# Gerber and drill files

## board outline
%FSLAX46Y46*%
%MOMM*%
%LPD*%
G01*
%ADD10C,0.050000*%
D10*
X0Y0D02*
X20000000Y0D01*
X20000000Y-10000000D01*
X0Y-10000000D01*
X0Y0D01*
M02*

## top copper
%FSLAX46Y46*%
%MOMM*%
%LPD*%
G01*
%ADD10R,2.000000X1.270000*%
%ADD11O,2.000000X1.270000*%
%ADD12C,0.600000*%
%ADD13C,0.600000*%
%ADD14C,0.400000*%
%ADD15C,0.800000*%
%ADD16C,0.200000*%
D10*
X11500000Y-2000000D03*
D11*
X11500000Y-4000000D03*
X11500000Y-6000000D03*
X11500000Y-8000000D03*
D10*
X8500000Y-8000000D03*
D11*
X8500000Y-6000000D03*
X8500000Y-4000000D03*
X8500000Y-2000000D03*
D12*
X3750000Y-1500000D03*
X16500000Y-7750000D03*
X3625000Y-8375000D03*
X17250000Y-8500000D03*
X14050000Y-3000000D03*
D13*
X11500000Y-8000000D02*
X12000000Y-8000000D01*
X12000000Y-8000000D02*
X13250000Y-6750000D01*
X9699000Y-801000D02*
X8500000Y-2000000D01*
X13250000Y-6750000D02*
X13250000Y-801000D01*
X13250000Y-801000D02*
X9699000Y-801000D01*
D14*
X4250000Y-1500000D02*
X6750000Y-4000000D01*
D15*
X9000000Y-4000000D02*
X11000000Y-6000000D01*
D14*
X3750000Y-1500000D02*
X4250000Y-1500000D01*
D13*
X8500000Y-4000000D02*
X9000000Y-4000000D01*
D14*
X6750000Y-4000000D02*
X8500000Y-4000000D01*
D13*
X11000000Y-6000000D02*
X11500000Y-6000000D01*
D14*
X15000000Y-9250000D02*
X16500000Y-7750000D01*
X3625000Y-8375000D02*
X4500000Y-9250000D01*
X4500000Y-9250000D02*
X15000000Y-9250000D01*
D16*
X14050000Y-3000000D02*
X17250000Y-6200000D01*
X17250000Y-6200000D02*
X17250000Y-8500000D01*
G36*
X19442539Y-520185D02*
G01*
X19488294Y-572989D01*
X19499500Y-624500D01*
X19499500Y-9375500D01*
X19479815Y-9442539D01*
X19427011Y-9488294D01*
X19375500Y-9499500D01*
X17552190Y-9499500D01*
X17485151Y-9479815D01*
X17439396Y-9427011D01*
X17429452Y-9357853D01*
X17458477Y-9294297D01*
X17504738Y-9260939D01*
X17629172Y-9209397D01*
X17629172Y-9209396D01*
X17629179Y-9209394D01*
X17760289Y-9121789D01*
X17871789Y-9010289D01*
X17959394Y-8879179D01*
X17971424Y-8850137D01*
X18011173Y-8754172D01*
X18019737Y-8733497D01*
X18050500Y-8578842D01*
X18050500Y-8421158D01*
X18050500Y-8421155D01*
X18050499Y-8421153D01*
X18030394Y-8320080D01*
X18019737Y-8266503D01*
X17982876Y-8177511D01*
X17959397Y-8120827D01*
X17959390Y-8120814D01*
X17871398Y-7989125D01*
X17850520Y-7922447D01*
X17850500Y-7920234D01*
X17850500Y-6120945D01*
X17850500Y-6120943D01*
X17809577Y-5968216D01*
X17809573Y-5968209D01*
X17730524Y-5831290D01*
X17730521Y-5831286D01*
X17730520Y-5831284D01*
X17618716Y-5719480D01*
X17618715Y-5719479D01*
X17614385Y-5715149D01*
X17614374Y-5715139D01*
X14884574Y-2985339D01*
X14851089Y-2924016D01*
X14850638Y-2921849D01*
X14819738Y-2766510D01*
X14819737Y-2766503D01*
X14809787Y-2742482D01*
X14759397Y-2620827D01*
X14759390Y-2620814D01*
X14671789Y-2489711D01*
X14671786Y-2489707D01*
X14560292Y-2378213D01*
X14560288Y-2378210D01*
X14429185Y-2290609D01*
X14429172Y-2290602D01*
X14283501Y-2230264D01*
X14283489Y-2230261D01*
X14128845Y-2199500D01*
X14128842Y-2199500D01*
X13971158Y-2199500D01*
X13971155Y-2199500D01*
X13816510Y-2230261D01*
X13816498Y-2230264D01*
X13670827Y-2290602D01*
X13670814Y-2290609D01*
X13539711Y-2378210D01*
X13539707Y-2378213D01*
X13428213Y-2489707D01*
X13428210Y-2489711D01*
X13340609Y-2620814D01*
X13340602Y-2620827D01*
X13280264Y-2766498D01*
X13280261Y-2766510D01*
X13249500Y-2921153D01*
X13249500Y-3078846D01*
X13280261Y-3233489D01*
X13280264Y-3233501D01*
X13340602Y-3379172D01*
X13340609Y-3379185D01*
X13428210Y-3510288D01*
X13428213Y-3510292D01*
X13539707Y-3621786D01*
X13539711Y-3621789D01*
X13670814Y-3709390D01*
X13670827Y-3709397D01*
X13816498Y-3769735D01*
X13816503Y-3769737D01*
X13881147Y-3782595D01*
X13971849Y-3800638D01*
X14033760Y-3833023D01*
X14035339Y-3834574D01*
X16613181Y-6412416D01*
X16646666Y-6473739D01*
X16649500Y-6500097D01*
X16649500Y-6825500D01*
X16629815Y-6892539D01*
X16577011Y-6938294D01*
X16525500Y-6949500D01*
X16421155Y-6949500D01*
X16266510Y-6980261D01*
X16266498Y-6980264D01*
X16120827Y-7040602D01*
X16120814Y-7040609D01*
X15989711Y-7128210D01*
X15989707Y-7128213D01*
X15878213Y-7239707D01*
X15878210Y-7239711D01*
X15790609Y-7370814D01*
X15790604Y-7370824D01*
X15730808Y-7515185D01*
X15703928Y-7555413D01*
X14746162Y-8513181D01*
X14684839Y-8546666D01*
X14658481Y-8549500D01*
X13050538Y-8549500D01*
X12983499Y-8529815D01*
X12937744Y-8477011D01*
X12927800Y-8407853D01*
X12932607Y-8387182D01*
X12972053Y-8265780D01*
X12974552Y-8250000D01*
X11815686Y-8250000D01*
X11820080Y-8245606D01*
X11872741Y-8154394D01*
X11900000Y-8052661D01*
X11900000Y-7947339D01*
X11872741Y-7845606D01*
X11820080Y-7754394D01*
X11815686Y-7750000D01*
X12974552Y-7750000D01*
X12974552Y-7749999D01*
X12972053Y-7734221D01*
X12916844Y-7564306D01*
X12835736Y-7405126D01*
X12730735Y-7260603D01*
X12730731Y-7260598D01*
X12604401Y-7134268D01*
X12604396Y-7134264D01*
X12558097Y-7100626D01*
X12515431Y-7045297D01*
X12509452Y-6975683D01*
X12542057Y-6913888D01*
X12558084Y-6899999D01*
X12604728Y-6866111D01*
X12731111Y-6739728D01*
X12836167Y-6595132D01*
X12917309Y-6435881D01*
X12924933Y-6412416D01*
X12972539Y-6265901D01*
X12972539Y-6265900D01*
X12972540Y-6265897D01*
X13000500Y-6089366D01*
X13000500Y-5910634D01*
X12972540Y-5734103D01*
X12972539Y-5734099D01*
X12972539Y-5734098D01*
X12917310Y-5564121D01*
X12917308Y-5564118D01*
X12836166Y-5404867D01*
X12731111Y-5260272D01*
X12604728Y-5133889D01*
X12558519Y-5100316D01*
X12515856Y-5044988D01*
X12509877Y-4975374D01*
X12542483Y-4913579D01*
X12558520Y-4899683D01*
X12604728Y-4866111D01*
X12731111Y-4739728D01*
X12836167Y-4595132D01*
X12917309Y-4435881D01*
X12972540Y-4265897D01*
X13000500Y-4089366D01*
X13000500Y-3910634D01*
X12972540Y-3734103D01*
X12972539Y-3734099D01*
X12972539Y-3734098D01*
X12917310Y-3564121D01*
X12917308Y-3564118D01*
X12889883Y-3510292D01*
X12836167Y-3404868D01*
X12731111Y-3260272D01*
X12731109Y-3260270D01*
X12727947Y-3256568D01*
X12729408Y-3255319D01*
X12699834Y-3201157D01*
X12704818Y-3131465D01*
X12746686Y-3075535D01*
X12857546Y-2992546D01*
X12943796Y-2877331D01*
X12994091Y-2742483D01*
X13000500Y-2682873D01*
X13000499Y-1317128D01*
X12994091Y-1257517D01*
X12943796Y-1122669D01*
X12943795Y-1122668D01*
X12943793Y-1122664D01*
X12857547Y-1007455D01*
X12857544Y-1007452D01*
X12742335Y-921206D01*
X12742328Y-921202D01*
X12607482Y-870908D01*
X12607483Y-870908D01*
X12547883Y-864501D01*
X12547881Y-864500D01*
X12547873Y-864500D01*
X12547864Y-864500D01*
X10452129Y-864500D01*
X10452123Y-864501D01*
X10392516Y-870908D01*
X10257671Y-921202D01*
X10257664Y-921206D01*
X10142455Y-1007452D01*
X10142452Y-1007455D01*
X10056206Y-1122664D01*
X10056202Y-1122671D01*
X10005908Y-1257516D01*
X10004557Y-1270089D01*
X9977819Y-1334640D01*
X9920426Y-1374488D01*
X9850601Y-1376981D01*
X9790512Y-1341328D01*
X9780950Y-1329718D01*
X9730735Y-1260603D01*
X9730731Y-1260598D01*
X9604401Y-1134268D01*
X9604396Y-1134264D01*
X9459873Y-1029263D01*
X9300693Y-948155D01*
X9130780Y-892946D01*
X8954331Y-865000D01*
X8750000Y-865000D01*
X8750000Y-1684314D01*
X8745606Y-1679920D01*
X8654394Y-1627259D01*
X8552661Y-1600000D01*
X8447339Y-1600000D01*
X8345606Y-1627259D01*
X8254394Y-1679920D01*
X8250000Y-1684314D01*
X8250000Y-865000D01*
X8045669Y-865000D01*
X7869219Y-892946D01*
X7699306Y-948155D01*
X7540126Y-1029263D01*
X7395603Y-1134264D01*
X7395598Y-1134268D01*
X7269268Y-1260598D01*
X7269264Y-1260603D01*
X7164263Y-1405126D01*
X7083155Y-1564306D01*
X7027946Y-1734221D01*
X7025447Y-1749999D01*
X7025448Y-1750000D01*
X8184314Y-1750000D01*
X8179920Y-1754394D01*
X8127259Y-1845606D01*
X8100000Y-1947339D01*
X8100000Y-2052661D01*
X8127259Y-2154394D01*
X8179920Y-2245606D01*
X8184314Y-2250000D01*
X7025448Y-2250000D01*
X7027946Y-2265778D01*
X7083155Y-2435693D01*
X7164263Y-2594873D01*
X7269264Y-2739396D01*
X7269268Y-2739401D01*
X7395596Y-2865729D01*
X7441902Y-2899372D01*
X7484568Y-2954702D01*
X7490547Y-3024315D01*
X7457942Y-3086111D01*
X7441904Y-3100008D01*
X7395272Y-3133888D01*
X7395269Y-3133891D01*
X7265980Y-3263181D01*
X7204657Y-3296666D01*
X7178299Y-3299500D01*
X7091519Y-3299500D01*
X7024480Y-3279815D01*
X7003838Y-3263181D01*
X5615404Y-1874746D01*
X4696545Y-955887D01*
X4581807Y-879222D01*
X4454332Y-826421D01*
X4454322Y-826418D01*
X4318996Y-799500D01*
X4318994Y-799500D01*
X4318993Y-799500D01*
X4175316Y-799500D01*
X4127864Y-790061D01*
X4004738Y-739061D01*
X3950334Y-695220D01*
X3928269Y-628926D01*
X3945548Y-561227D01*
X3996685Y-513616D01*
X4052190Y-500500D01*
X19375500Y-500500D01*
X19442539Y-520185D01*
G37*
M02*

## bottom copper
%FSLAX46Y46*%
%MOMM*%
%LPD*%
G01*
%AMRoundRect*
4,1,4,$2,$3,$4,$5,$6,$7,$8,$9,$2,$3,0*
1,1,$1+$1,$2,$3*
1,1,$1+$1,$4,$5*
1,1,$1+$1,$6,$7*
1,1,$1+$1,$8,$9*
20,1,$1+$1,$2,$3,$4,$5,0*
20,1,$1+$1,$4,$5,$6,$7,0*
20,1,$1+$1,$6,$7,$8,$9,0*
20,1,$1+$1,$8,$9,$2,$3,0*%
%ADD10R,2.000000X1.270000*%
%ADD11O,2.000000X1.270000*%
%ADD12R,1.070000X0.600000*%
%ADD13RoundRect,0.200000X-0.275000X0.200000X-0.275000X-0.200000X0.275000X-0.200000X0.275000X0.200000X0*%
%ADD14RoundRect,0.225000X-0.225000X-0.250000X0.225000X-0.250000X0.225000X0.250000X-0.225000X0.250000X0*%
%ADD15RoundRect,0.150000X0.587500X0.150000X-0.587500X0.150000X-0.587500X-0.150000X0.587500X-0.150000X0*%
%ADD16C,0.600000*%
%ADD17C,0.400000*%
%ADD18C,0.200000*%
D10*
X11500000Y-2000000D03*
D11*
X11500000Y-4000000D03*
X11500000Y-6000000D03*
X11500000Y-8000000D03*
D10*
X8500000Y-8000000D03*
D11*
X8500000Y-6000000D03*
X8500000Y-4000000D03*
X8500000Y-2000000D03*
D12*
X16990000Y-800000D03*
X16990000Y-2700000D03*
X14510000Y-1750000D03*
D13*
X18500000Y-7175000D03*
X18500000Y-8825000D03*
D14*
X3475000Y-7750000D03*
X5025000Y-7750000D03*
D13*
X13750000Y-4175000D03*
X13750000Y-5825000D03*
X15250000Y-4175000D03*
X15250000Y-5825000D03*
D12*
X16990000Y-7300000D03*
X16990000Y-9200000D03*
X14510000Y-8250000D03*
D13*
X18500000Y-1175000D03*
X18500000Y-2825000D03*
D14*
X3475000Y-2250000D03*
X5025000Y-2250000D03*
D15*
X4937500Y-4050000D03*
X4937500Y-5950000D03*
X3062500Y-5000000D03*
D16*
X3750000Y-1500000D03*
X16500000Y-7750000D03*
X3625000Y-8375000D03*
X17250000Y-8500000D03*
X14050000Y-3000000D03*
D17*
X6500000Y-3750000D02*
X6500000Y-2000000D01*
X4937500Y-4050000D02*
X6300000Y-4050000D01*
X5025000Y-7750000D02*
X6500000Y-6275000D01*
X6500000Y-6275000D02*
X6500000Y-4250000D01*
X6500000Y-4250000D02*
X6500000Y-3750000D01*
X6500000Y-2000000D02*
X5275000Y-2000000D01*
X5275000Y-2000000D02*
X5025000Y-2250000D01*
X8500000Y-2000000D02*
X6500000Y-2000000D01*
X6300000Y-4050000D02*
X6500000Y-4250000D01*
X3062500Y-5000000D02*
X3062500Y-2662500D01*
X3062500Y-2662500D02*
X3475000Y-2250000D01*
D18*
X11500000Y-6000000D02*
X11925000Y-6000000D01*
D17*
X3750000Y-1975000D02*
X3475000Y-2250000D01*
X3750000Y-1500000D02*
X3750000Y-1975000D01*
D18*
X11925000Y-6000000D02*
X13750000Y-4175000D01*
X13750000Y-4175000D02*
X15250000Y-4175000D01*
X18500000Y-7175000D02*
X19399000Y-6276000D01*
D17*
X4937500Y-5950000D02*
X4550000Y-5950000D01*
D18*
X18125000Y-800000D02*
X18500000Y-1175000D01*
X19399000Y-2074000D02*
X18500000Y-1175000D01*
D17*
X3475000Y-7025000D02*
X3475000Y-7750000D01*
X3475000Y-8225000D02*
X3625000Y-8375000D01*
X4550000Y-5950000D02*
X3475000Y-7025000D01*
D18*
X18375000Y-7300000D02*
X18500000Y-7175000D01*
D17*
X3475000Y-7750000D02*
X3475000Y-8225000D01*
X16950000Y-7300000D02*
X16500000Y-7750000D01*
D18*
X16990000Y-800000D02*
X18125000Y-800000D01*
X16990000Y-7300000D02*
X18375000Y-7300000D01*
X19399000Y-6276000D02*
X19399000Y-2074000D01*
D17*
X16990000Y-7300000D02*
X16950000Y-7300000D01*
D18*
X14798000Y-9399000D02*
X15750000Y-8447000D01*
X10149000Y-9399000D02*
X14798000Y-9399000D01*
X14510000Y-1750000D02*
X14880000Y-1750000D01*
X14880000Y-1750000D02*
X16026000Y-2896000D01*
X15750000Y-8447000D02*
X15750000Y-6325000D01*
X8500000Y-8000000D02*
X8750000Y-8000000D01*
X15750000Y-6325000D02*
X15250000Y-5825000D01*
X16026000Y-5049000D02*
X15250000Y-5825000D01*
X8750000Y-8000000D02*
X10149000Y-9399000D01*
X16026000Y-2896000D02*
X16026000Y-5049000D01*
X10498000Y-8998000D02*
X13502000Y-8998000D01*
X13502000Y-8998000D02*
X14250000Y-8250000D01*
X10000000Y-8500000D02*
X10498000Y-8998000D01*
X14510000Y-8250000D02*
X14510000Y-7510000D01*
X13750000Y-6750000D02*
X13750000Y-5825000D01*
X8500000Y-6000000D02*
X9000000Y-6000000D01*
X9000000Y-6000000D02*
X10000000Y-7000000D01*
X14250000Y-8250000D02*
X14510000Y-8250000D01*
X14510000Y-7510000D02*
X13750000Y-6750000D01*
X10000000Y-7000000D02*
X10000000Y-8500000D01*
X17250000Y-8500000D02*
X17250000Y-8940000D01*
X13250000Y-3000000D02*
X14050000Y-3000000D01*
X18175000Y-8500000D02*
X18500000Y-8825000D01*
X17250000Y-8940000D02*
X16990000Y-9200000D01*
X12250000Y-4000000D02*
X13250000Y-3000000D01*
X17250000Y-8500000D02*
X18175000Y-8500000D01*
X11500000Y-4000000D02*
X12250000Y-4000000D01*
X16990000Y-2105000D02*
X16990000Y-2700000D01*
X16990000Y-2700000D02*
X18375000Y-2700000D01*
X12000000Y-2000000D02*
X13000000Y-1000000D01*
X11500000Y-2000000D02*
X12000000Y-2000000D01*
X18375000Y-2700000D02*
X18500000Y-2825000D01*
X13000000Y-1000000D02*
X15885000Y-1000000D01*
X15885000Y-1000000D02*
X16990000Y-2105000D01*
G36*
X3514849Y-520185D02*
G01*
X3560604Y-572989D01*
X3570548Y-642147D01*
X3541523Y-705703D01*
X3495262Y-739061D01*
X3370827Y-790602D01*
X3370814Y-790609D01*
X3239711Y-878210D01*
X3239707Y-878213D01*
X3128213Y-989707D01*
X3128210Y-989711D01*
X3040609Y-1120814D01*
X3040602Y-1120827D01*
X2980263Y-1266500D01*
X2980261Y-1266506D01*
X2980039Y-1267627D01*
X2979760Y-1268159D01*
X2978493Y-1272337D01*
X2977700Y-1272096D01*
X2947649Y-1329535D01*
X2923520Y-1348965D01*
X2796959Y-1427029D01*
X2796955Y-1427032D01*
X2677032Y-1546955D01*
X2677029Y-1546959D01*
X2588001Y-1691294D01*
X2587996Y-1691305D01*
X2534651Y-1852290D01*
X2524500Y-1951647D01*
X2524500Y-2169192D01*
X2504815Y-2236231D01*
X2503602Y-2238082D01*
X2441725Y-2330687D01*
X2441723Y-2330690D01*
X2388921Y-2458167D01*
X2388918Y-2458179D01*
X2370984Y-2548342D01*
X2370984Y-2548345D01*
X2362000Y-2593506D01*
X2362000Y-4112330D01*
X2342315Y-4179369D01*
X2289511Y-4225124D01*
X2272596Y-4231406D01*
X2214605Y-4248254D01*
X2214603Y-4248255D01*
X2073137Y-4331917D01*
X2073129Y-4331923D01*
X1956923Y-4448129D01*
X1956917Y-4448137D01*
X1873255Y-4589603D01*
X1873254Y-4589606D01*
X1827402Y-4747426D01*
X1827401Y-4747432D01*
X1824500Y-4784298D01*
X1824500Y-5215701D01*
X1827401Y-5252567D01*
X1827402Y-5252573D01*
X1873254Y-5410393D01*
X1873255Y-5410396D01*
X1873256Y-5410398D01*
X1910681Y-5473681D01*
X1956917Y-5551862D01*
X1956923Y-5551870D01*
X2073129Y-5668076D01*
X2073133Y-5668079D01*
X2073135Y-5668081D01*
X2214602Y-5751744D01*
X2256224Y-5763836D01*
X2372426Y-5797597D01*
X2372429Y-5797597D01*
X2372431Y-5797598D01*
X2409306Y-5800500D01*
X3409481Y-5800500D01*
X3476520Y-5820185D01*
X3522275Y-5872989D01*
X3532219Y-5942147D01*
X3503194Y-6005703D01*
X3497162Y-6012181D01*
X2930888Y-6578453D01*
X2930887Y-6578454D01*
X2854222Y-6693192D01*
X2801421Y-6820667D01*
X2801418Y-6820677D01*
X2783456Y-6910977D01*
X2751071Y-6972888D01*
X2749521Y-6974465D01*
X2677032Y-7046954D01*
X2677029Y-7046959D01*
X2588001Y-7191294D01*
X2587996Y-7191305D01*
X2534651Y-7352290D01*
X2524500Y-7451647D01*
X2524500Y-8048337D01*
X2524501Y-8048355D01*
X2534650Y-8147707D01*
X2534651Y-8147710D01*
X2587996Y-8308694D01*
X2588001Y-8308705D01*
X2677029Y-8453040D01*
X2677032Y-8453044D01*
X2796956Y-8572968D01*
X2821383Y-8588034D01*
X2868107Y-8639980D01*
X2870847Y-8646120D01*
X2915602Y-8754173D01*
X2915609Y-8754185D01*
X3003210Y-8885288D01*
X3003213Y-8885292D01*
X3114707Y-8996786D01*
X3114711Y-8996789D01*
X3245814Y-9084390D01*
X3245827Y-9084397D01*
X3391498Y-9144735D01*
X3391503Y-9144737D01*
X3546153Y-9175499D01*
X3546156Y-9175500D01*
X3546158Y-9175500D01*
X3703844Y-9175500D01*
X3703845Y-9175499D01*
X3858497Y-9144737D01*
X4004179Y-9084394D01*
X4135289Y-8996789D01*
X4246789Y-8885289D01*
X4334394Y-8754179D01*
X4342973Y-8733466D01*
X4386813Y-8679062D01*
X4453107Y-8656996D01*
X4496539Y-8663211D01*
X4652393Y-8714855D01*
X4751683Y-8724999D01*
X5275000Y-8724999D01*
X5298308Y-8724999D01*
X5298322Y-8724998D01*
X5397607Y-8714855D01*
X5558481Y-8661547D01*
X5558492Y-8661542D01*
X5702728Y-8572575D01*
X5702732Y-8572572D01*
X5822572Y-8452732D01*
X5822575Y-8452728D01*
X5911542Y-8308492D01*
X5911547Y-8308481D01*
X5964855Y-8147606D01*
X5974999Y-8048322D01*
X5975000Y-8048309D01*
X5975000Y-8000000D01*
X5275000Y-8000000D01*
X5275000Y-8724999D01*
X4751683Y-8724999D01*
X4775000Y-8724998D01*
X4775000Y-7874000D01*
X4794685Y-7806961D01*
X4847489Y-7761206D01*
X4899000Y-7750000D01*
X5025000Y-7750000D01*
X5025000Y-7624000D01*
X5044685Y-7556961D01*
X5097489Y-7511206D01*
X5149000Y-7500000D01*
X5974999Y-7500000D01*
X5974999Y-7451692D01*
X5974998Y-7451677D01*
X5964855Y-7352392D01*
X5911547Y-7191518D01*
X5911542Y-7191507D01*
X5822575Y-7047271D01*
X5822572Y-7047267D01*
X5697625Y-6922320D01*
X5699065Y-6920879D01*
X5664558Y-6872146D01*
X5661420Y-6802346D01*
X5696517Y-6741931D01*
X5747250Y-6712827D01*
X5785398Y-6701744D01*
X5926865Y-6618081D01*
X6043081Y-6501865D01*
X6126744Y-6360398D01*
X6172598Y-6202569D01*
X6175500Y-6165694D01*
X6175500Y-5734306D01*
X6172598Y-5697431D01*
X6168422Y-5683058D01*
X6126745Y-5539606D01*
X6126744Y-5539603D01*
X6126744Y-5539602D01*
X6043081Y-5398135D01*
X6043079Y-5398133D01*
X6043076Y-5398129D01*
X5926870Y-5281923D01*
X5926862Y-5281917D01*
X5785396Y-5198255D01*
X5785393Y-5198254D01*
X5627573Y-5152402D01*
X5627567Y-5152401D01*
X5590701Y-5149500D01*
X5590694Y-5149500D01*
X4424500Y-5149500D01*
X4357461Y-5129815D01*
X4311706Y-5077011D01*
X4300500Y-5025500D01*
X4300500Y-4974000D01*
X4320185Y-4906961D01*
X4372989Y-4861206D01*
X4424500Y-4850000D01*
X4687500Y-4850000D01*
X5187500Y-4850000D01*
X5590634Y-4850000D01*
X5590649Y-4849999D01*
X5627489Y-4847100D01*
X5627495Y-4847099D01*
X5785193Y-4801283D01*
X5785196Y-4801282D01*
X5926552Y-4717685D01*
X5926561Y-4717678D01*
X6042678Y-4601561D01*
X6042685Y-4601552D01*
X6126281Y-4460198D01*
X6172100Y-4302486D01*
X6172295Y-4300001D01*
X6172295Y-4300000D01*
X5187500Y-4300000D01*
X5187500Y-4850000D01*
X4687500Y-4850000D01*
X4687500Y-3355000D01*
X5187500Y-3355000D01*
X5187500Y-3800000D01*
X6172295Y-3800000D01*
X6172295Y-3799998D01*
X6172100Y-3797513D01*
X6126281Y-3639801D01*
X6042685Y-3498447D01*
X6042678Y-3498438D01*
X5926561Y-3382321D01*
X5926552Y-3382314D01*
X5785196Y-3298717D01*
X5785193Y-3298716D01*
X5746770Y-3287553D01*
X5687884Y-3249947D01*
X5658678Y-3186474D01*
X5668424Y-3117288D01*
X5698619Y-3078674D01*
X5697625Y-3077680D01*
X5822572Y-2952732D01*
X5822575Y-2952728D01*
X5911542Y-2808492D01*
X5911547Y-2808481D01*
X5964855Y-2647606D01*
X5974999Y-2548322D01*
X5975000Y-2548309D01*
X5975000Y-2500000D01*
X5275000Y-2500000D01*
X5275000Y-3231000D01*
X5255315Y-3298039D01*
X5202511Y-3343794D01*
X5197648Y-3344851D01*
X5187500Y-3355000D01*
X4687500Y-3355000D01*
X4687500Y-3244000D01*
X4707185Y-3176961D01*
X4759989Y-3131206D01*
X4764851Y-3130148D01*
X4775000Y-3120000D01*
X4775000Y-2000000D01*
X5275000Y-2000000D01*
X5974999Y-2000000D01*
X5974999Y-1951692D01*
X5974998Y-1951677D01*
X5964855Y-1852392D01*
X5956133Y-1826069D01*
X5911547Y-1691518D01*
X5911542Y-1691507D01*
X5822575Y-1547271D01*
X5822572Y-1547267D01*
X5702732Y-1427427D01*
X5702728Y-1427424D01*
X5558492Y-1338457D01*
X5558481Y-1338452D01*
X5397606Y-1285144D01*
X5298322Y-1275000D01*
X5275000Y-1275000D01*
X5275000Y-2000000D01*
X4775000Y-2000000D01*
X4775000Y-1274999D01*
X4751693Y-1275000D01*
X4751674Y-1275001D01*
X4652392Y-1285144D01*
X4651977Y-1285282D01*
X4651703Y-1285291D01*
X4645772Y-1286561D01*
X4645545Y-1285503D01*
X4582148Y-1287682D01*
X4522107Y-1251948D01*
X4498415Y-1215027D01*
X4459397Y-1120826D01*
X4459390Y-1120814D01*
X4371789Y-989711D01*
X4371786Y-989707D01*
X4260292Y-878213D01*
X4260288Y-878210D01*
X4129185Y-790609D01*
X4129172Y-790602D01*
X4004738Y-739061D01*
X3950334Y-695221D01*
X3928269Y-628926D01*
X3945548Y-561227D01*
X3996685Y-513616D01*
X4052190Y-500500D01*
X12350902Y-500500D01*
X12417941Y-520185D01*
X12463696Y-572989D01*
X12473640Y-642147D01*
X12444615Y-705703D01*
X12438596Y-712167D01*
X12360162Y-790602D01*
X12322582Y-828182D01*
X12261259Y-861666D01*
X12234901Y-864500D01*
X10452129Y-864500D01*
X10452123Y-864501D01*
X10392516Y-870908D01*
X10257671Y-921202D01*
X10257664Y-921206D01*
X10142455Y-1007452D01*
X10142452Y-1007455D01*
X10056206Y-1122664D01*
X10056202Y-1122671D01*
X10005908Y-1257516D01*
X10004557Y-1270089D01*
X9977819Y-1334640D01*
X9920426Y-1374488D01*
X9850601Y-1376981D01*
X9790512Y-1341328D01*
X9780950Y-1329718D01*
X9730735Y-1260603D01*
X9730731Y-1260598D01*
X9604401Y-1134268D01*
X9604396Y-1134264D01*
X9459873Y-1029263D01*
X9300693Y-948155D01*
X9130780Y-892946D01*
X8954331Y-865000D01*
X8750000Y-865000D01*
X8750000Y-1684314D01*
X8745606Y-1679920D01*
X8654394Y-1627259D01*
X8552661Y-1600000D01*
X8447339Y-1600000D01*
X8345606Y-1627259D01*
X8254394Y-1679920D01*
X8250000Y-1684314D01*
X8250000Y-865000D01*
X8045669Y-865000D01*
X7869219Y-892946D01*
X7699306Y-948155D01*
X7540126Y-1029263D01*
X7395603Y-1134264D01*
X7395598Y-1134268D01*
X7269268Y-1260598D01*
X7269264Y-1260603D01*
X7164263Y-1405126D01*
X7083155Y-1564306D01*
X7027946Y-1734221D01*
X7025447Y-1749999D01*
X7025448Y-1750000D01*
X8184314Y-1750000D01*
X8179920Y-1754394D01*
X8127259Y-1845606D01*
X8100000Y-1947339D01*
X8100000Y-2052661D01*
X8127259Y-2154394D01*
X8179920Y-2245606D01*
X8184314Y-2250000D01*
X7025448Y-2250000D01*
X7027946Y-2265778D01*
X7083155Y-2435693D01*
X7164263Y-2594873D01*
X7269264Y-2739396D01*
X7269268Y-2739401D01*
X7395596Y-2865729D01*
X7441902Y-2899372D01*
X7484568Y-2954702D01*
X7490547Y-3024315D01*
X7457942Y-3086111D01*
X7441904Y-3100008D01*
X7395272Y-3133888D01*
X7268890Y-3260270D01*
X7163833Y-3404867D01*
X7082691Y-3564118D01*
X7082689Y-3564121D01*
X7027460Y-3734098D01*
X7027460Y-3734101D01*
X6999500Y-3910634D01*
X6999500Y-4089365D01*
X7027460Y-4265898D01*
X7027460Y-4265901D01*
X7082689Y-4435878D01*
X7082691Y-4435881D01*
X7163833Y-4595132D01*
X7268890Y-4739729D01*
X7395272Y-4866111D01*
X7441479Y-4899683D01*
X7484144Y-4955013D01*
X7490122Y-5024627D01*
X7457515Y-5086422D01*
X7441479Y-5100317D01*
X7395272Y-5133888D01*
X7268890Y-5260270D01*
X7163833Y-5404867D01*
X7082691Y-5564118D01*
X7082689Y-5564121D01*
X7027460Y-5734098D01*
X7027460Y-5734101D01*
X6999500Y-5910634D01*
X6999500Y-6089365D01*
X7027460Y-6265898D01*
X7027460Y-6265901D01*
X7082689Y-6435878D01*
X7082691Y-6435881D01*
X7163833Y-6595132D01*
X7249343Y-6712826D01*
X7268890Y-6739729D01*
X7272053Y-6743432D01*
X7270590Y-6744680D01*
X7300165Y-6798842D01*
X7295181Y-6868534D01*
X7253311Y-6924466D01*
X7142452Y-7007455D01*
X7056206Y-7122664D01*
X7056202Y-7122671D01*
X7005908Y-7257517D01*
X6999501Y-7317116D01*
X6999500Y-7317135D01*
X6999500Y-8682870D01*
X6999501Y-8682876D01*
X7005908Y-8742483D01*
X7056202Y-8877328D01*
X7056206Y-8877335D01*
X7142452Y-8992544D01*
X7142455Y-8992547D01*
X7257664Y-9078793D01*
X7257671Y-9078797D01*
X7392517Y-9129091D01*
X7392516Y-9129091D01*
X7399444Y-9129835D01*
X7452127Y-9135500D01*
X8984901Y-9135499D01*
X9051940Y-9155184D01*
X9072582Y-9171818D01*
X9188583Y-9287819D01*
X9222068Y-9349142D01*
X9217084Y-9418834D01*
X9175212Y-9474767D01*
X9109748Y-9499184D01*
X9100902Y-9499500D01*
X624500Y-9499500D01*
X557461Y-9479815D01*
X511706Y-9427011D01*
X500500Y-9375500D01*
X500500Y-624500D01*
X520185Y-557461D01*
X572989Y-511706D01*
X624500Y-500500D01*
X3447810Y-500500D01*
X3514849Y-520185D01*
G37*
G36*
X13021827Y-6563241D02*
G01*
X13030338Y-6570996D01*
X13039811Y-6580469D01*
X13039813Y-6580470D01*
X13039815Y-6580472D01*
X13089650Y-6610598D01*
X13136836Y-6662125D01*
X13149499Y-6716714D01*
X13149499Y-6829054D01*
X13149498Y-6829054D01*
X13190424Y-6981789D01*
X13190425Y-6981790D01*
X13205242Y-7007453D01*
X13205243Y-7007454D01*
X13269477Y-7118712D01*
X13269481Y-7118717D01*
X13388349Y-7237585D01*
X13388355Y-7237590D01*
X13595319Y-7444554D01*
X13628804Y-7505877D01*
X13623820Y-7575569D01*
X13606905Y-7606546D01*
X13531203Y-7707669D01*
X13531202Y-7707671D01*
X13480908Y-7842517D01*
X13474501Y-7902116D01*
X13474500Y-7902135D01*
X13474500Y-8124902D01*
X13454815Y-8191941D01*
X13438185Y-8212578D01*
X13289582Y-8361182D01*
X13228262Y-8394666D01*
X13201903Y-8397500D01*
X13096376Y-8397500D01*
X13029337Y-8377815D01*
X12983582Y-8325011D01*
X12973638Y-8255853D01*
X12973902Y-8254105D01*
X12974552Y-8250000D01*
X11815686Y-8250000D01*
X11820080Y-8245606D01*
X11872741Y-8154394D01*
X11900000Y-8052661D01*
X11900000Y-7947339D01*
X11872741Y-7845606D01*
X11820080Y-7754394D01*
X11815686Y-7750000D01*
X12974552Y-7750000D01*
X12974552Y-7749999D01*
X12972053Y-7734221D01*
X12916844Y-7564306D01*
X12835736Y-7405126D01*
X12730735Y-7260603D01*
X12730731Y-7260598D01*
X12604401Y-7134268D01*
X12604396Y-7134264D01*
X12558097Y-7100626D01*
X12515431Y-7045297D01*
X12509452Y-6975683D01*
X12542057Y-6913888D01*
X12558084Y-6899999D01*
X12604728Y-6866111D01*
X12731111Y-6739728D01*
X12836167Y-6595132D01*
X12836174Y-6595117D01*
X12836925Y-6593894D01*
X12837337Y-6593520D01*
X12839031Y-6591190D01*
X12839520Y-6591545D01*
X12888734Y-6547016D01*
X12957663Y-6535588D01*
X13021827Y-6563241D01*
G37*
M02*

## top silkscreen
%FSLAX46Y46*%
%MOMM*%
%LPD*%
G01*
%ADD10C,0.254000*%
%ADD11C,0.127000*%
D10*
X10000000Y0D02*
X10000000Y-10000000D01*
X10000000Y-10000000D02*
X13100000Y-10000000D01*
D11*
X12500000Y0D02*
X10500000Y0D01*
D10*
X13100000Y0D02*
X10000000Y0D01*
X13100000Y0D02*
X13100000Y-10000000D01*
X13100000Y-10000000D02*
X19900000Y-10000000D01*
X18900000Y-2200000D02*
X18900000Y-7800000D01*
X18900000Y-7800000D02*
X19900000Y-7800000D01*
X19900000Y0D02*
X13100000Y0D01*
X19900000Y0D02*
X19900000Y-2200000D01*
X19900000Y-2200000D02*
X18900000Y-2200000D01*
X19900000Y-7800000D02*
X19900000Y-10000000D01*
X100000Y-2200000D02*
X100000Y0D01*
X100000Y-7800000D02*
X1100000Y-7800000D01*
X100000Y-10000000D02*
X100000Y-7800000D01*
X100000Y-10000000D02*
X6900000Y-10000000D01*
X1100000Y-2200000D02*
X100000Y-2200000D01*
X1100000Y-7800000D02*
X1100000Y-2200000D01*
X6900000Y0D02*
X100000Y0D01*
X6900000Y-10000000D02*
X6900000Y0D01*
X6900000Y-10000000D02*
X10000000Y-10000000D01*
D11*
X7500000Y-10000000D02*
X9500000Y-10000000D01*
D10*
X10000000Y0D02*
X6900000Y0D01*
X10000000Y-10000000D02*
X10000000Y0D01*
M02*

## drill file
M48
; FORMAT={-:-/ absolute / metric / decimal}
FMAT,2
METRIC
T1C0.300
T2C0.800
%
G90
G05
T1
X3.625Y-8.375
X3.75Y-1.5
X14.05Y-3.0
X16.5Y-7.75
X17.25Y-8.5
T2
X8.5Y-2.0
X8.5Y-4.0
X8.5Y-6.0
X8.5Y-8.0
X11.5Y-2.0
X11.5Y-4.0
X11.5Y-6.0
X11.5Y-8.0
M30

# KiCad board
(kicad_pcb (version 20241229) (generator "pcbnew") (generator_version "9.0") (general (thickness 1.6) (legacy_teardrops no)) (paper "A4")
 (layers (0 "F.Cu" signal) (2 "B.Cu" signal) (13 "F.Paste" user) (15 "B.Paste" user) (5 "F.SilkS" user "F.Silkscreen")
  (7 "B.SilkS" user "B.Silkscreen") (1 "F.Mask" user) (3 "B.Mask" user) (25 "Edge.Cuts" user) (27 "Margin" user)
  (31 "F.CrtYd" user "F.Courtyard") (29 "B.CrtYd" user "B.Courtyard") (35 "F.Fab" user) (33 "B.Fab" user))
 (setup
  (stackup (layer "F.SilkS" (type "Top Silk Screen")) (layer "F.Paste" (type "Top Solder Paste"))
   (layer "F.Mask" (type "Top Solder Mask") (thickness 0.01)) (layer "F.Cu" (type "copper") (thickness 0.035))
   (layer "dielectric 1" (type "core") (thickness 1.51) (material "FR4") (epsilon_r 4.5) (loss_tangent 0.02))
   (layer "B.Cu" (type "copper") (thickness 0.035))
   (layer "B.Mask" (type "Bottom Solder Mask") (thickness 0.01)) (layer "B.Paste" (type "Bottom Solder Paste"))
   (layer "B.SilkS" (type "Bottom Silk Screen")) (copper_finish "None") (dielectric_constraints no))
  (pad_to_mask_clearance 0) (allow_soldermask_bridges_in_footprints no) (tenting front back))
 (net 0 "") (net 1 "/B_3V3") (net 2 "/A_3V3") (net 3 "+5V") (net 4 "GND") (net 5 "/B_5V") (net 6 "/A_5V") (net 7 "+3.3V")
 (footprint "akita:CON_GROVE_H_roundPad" (layer "F.Cu") (at 11.5 5 -90)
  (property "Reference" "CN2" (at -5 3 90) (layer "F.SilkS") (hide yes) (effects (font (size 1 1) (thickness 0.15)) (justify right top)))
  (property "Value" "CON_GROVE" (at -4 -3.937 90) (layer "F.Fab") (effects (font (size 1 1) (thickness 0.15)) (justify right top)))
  (fp_line (start -5 1.5) (end 5 1.5) (stroke (width 0.254) (type solid)) (layer "F.SilkS"))
  (fp_line (start 5 1.5) (end 5 -1.6) (stroke (width 0.254) (type solid)) (layer "F.SilkS"))
  (fp_line (start -5 -1) (end -5 1) (stroke (width 0.127) (type solid)) (layer "F.SilkS"))
  (fp_line (start -5 -1.6) (end -5 1.5) (stroke (width 0.254) (type solid)) (layer "F.SilkS"))
  (fp_line (start -5 -1.6) (end 5 -1.6) (stroke (width 0.254) (type solid)) (layer "F.SilkS"))
  (fp_line (start 5 -1.6) (end 5 -8.4) (stroke (width 0.254) (type solid)) (layer "F.SilkS"))
  (fp_line (start -2.8 -7.4) (end 2.8 -7.4) (stroke (width 0.254) (type solid)) (layer "F.SilkS"))
  (fp_line (start 2.8 -7.4) (end 2.8 -8.4) (stroke (width 0.254) (type solid)) (layer "F.SilkS"))
  (fp_line (start -5 -8.4) (end -5 -1.6) (stroke (width 0.254) (type solid)) (layer "F.SilkS"))
  (fp_line (start -5 -8.4) (end -2.8 -8.4) (stroke (width 0.254) (type solid)) (layer "F.SilkS"))
  (fp_line (start -2.8 -8.4) (end -2.8 -7.4) (stroke (width 0.254) (type solid)) (layer "F.SilkS"))
  (fp_line (start 2.8 -8.4) (end 5 -8.4) (stroke (width 0.254) (type solid)) (layer "F.SilkS"))
  (pad "1" thru_hole rect (at -3 0 270) (size 1.27 2) (drill 0.8) (layers "*.Cu" "*.Mask") (remove_unused_layers no) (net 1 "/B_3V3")
   (solder_mask_margin 0.1016))
  (pad "2" thru_hole oval (at -1 0 270) (size 1.27 2) (drill 0.8) (layers "*.Cu" "*.Mask") (remove_unused_layers no) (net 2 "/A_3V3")
   (solder_mask_margin 0.1016))
  (pad "3" thru_hole oval (at 1 0 270) (size 1.27 2) (drill 0.8) (layers "*.Cu" "*.Mask") (remove_unused_layers no) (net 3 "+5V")
   (solder_mask_margin 0.1016))
  (pad "4" thru_hole oval (at 3 0 270) (size 1.27 2) (drill 0.8) (layers "*.Cu" "*.Mask") (remove_unused_layers no) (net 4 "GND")
   (solder_mask_margin 0.1016)))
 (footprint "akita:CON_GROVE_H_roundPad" (layer "F.Cu") (at 8.5 5 90)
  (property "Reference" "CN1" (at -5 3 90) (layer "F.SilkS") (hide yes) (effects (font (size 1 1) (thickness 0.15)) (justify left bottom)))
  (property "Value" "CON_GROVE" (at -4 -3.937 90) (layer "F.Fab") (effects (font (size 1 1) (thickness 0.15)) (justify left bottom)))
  (fp_line (start 2.8 -8.4) (end 5 -8.4) (stroke (width 0.254) (type solid)) (layer "F.SilkS"))
  (fp_line (start -2.8 -8.4) (end -2.8 -7.4) (stroke (width 0.254) (type solid)) (layer "F.SilkS"))
  (fp_line (start -5 -8.4) (end -2.8 -8.4) (stroke (width 0.254) (type solid)) (layer "F.SilkS"))
  (fp_line (start -5 -8.4) (end -5 -1.6) (stroke (width 0.254) (type solid)) (layer "F.SilkS"))
  (fp_line (start 2.8 -7.4) (end 2.8 -8.4) (stroke (width 0.254) (type solid)) (layer "F.SilkS"))
  (fp_line (start -2.8 -7.4) (end 2.8 -7.4) (stroke (width 0.254) (type solid)) (layer "F.SilkS"))
  (fp_line (start 5 -1.6) (end 5 -8.4) (stroke (width 0.254) (type solid)) (layer "F.SilkS"))
  (fp_line (start -5 -1.6) (end 5 -1.6) (stroke (width 0.254) (type solid)) (layer "F.SilkS"))
  (fp_line (start -5 -1.6) (end -5 1.5) (stroke (width 0.254) (type solid)) (layer "F.SilkS"))
  (fp_line (start -5 -1) (end -5 1) (stroke (width 0.127) (type solid)) (layer "F.SilkS"))
  (fp_line (start 5 1.5) (end 5 -1.6) (stroke (width 0.254) (type solid)) (layer "F.SilkS"))
  (fp_line (start -5 1.5) (end 5 1.5) (stroke (width 0.254) (type solid)) (layer "F.SilkS"))
  (pad "1" thru_hole rect (at -3 0 90) (size 1.27 2) (drill 0.8) (layers "*.Cu" "*.Mask") (remove_unused_layers no) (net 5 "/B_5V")
   (solder_mask_margin 0.1016))
  (pad "2" thru_hole oval (at -1 0 90) (size 1.27 2) (drill 0.8) (layers "*.Cu" "*.Mask") (remove_unused_layers no) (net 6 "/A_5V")
   (solder_mask_margin 0.1016))
  (pad "3" thru_hole oval (at 1 0 90) (size 1.27 2) (drill 0.8) (layers "*.Cu" "*.Mask") (remove_unused_layers no) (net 3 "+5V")
   (solder_mask_margin 0.1016))
  (pad "4" thru_hole oval (at 3 0 90) (size 1.27 2) (drill 0.8) (layers "*.Cu" "*.Mask") (remove_unused_layers no) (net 4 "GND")
   (solder_mask_margin 0.1016)))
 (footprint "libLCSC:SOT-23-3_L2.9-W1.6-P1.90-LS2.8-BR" (layer "B.Cu") (at 15.75 1.75)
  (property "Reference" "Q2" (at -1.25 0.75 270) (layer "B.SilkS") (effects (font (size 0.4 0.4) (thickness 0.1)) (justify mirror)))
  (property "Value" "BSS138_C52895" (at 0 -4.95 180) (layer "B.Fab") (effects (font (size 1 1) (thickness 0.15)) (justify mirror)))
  (pad "1" smd rect (at 1.24 -0.95) (size 1.07 0.6) (layers "B.Cu" "B.Mask" "B.Paste") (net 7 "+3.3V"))
  (pad "2" smd rect (at 1.24 0.95) (size 1.07 0.6) (layers "B.Cu" "B.Mask" "B.Paste") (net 1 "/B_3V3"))
  (pad "3" smd rect (at -1.24 0) (size 1.07 0.6) (layers "B.Cu" "B.Mask" "B.Paste") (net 5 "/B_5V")))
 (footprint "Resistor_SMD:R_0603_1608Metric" (layer "B.Cu") (at 18.5 8 -90)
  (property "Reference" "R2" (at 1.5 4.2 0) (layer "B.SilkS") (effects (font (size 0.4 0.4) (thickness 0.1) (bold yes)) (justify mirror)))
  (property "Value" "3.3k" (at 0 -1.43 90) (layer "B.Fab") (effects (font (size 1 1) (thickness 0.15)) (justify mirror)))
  (pad "1" smd roundrect (at -0.825 0 270) (size 0.8 0.95) (layers "B.Cu" "B.Mask" "B.Paste") (roundrect_rratio 0.25) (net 7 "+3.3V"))
  (pad "2" smd roundrect (at 0.825 0 270) (size 0.8 0.95) (layers "B.Cu" "B.Mask" "B.Paste") (roundrect_rratio 0.25) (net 2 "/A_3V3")))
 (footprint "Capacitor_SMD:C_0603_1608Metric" (layer "B.Cu") (at 4.25 7.75)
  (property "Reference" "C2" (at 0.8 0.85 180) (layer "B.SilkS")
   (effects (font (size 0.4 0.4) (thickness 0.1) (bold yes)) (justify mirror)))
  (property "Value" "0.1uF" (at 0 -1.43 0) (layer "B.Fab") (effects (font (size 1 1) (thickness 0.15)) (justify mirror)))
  (pad "1" smd roundrect (at -0.775 0) (size 0.9 0.95) (layers "B.Cu" "B.Mask" "B.Paste") (roundrect_rratio 0.25) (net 7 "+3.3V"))
  (pad "2" smd roundrect (at 0.775 0) (size 0.9 0.95) (layers "B.Cu" "B.Mask" "B.Paste") (roundrect_rratio 0.25) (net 4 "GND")))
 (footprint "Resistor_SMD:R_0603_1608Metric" (layer "B.Cu") (at 13.75 5 -90)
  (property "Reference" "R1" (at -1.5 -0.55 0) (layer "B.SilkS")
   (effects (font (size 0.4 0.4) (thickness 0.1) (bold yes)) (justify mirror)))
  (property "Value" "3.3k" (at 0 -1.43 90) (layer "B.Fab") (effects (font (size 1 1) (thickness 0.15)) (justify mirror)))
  (pad "1" smd roundrect (at -0.825 0 270) (size 0.8 0.95) (layers "B.Cu" "B.Mask" "B.Paste") (roundrect_rratio 0.25) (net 3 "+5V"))
  (pad "2" smd roundrect (at 0.825 0 270) (size 0.8 0.95) (layers "B.Cu" "B.Mask" "B.Paste") (roundrect_rratio 0.25) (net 6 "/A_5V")))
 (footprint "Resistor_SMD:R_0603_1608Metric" (layer "B.Cu") (at 15.25 5 -90)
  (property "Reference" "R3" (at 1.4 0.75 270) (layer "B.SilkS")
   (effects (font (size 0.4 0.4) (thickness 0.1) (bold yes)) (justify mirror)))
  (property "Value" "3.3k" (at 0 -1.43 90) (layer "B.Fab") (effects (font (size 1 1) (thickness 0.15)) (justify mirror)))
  (pad "1" smd roundrect (at -0.825 0 270) (size 0.8 0.95) (layers "B.Cu" "B.Mask" "B.Paste") (roundrect_rratio 0.25) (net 3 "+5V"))
  (pad "2" smd roundrect (at 0.825 0 270) (size 0.8 0.95) (layers "B.Cu" "B.Mask" "B.Paste") (roundrect_rratio 0.25) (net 5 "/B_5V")))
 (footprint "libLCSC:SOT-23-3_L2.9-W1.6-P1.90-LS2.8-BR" (layer "B.Cu") (at 15.75 8.25)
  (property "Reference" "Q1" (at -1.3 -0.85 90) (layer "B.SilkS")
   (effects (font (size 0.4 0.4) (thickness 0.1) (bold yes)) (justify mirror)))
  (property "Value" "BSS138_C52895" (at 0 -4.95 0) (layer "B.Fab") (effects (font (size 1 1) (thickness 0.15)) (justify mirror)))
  (pad "1" smd rect (at 1.24 -0.95) (size 1.07 0.6) (layers "B.Cu" "B.Mask" "B.Paste") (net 7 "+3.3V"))
  (pad "2" smd rect (at 1.24 0.95) (size 1.07 0.6) (layers "B.Cu" "B.Mask" "B.Paste") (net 2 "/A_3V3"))
  (pad "3" smd rect (at -1.24 0) (size 1.07 0.6) (layers "B.Cu" "B.Mask" "B.Paste") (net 6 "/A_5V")))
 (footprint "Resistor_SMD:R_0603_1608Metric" (layer "B.Cu") (at 18.5 2 -90)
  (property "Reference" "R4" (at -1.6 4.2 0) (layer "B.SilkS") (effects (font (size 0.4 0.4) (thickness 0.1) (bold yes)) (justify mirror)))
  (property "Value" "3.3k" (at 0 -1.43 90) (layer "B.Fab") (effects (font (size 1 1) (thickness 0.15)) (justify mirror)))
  (pad "1" smd roundrect (at -0.825 0 270) (size 0.8 0.95) (layers "B.Cu" "B.Mask" "B.Paste") (roundrect_rratio 0.25) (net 7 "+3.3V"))
  (pad "2" smd roundrect (at 0.825 0 270) (size 0.8 0.95) (layers "B.Cu" "B.Mask" "B.Paste") (roundrect_rratio 0.25) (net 1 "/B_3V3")))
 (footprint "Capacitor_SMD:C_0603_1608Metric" (layer "B.Cu") (at 4.25 2.25)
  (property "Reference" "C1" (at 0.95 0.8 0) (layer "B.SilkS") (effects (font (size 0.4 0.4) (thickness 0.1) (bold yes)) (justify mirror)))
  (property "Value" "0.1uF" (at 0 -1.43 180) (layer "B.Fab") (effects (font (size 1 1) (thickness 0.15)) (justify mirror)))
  (pad "1" smd roundrect (at -0.775 0) (size 0.9 0.95) (layers "B.Cu" "B.Mask" "B.Paste") (roundrect_rratio 0.25) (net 3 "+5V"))
  (pad "2" smd roundrect (at 0.775 0) (size 0.9 0.95) (layers "B.Cu" "B.Mask" "B.Paste") (roundrect_rratio 0.25) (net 4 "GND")))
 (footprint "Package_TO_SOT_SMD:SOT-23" (layer "B.Cu") (at 4 5 180)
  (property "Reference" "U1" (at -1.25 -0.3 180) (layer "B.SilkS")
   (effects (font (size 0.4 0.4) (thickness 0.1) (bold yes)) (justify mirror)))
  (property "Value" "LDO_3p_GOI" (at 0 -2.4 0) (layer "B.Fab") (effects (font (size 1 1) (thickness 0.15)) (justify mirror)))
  (pad "1" smd roundrect (at -0.9375 0.95 180) (size 1.475 0.6) (layers "B.Cu" "B.Mask" "B.Paste") (roundrect_rratio 0.25) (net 4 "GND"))
  (pad "2" smd roundrect (at -0.9375 -0.95 180) (size 1.475 0.6) (layers "B.Cu" "B.Mask" "B.Paste") (roundrect_rratio 0.25) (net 7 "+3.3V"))
  (pad "3" smd roundrect (at 0.9375 0 180) (size 1.475 0.6) (layers "B.Cu" "B.Mask" "B.Paste") (roundrect_rratio 0.25) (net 3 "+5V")))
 (gr_rect (start 0 0) (end 20 10) (stroke (width 0.05) (type solid)) (fill no) (layer "Edge.Cuts"))
 (segment (start 11.5 8) (end 12 8) (width 0.6) (layer "F.Cu") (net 4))
 (segment (start 12 8) (end 13.25 6.75) (width 0.6) (layer "F.Cu") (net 4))
 (segment (start 9.699 0.801) (end 8.5 2) (width 0.6) (layer "F.Cu") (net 4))
 (segment (start 13.25 6.75) (end 13.25 0.801) (width 0.6) (layer "F.Cu") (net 4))
 (segment (start 13.25 0.801) (end 9.699 0.801) (width 0.6) (layer "F.Cu") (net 4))
 (segment (start 6.5 3.75) (end 6.5 2) (width 0.4) (layer "B.Cu") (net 4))
 (segment (start 4.9375 4.05) (end 6.3 4.05) (width 0.4) (layer "B.Cu") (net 4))
 (segment (start 5.025 7.75) (end 6.5 6.275) (width 0.4) (layer "B.Cu") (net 4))
 (segment (start 6.5 6.275) (end 6.5 4.25) (width 0.4) (layer "B.Cu") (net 4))
 (segment (start 6.5 4.25) (end 6.5 3.75) (width 0.4) (layer "B.Cu") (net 4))
 (segment (start 6.5 2) (end 5.275 2) (width 0.4) (layer "B.Cu") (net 4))
 (segment (start 5.275 2) (end 5.025 2.25) (width 0.4) (layer "B.Cu") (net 4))
 (segment (start 8.5 2) (end 6.5 2) (width 0.4) (layer "B.Cu") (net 4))
 (segment (start 6.3 4.05) (end 6.5 4.25) (width 0.4) (layer "B.Cu") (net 4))
 (segment (start 4.25 1.5) (end 6.75 4) (width 0.4) (layer "F.Cu") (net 3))
 (segment (start 9 4) (end 11 6) (width 0.8) (layer "F.Cu") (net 3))
 (segment (start 3.75 1.5) (end 4.25 1.5) (width 0.4) (layer "F.Cu") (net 3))
 (segment (start 8.5 4) (end 9 4) (width 0.6) (layer "F.Cu") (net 3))
 (segment (start 6.75 4) (end 8.5 4) (width 0.4) (layer "F.Cu") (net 3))
 (segment (start 11 6) (end 11.5 6) (width 0.6) (layer "F.Cu") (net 3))
 (via (at 3.75 1.5) (size 0.6) (drill 0.3) (layers "F.Cu" "B.Cu") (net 3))
 (segment (start 3.0625 5) (end 3.0625 2.6625) (width 0.4) (layer "B.Cu") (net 3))
 (segment (start 3.0625 2.6625) (end 3.475 2.25) (width 0.4) (layer "B.Cu") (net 3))
 (segment (start 11.5 6) (end 11.925 6) (width 0.2) (layer "B.Cu") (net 3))
 (segment (start 3.75 1.975) (end 3.475 2.25) (width 0.4) (layer "B.Cu") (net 3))
 (segment (start 3.75 1.5) (end 3.75 1.975) (width 0.4) (layer "B.Cu") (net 3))
 (segment (start 11.925 6) (end 13.75 4.175) (width 0.2) (layer "B.Cu") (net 3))
 (segment (start 13.75 4.175) (end 15.25 4.175) (width 0.2) (layer "B.Cu") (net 3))
 (segment (start 15 9.25) (end 16.5 7.75) (width 0.4) (layer "F.Cu") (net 7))
 (segment (start 3.625 8.375) (end 4.5 9.25) (width 0.4) (layer "F.Cu") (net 7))
 (segment (start 4.5 9.25) (end 15 9.25) (width 0.4) (layer "F.Cu") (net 7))
 (via (at 16.5 7.75) (size 0.6) (drill 0.3) (layers "F.Cu" "B.Cu") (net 7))
 (via (at 3.625 8.375) (size 0.6) (drill 0.3) (layers "F.Cu" "B.Cu") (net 7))
 (segment (start 18.5 7.175) (end 19.399 6.276) (width 0.2) (layer "B.Cu") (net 7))
 (segment (start 4.9375 5.95) (end 4.55 5.95) (width 0.4) (layer "B.Cu") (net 7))
 (segment (start 18.125 0.8) (end 18.5 1.175) (width 0.2) (layer "B.Cu") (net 7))
 (segment (start 19.399 2.074) (end 18.5 1.175) (width 0.2) (layer "B.Cu") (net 7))
 (segment (start 3.475 7.025) (end 3.475 7.75) (width 0.4) (layer "B.Cu") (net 7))
 (segment (start 3.475 8.225) (end 3.625 8.375) (width 0.4) (layer "B.Cu") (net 7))
 (segment (start 4.55 5.95) (end 3.475 7.025) (width 0.4) (layer "B.Cu") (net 7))
 (segment (start 18.375 7.3) (end 18.5 7.175) (width 0.2) (layer "B.Cu") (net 7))
 (segment (start 3.475 7.75) (end 3.475 8.225) (width 0.4) (layer "B.Cu") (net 7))
 (segment (start 16.95 7.3) (end 16.5 7.75) (width 0.4) (layer "B.Cu") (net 7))
 (segment (start 16.99 0.8) (end 18.125 0.8) (width 0.2) (layer "B.Cu") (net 7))
 (segment (start 16.99 7.3) (end 18.375 7.3) (width 0.2) (layer "B.Cu") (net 7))
 (segment (start 19.399 6.276) (end 19.399 2.074) (width 0.2) (layer "B.Cu") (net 7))
 (segment (start 16.99 7.3) (end 16.95 7.3) (width 0.4) (layer "B.Cu") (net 7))
 (segment (start 14.798 9.399) (end 15.75 8.447) (width 0.2) (layer "B.Cu") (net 5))
 (segment (start 10.149 9.399) (end 14.798 9.399) (width 0.2) (layer "B.Cu") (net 5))
 (segment (start 14.51 1.75) (end 14.88 1.75) (width 0.2) (layer "B.Cu") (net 5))
 (segment (start 14.88 1.75) (end 16.026 2.896) (width 0.2) (layer "B.Cu") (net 5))
 (segment (start 15.75 8.447) (end 15.75 6.325) (width 0.2) (layer "B.Cu") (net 5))
 (segment (start 8.5 8) (end 8.75 8) (width 0.2) (layer "B.Cu") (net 5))
 (segment (start 15.75 6.325) (end 15.25 5.825) (width 0.2) (layer "B.Cu") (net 5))
 (segment (start 16.026 5.049) (end 15.25 5.825) (width 0.2) (layer "B.Cu") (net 5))
 (segment (start 8.75 8) (end 10.149 9.399) (width 0.2) (layer "B.Cu") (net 5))
 (segment (start 16.026 2.896) (end 16.026 5.049) (width 0.2) (layer "B.Cu") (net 5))
 (segment (start 10.498 8.998) (end 13.502 8.998) (width 0.2) (layer "B.Cu") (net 6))
 (segment (start 13.502 8.998) (end 14.25 8.25) (width 0.2) (layer "B.Cu") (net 6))
 (segment (start 10 8.5) (end 10.498 8.998) (width 0.2) (layer "B.Cu") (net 6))
 (segment (start 14.51 8.25) (end 14.51 7.51) (width 0.2) (layer "B.Cu") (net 6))
 (segment (start 13.75 6.75) (end 13.75 5.825) (width 0.2) (layer "B.Cu") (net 6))
 (segment (start 8.5 6) (end 9 6) (width 0.2) (layer "B.Cu") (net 6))
 (segment (start 9 6) (end 10 7) (width 0.2) (layer "B.Cu") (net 6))
 (segment (start 14.25 8.25) (end 14.51 8.25) (width 0.2) (layer "B.Cu") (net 6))
 (segment (start 14.51 7.51) (end 13.75 6.75) (width 0.2) (layer "B.Cu") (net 6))
 (segment (start 10 7) (end 10 8.5) (width 0.2) (layer "B.Cu") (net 6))
 (segment (start 14.05 3) (end 17.25 6.2) (width 0.2) (layer "F.Cu") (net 2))
 (segment (start 17.25 6.2) (end 17.25 8.5) (width 0.2) (layer "F.Cu") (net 2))
 (via (at 17.25 8.5) (size 0.6) (drill 0.3) (layers "F.Cu" "B.Cu") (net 2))
 (via (at 14.05 3) (size 0.6) (drill 0.3) (layers "F.Cu" "B.Cu") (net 2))
 (segment (start 17.25 8.5) (end 17.25 8.94) (width 0.2) (layer "B.Cu") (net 2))
 (segment (start 13.25 3) (end 14.05 3) (width 0.2) (layer "B.Cu") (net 2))
 (segment (start 18.175 8.5) (end 18.5 8.825) (width 0.2) (layer "B.Cu") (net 2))
 (segment (start 17.25 8.94) (end 16.99 9.2) (width 0.2) (layer "B.Cu") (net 2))
 (segment (start 12.25 4) (end 13.25 3) (width 0.2) (layer "B.Cu") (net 2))
 (segment (start 17.25 8.5) (end 18.175 8.5) (width 0.2) (layer "B.Cu") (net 2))
 (segment (start 11.5 4) (end 12.25 4) (width 0.2) (layer "B.Cu") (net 2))
 (segment (start 16.99 2.105) (end 16.99 2.7) (width 0.2) (layer "B.Cu") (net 1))
 (segment (start 16.99 2.7) (end 18.375 2.7) (width 0.2) (layer "B.Cu") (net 1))
 (segment (start 12 2) (end 13 1) (width 0.2) (layer "B.Cu") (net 1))
 (segment (start 11.5 2) (end 12 2) (width 0.2) (layer "B.Cu") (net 1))
 (segment (start 18.375 2.7) (end 18.5 2.825) (width 0.2) (layer "B.Cu") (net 1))
 (segment (start 13 1) (end 15.885 1) (width 0.2) (layer "B.Cu") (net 1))
 (segment (start 15.885 1) (end 16.99 2.105) (width 0.2) (layer "B.Cu") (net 1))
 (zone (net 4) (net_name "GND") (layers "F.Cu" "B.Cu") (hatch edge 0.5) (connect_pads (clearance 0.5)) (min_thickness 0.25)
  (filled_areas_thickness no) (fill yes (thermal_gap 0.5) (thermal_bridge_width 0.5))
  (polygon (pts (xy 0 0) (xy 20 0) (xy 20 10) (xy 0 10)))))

